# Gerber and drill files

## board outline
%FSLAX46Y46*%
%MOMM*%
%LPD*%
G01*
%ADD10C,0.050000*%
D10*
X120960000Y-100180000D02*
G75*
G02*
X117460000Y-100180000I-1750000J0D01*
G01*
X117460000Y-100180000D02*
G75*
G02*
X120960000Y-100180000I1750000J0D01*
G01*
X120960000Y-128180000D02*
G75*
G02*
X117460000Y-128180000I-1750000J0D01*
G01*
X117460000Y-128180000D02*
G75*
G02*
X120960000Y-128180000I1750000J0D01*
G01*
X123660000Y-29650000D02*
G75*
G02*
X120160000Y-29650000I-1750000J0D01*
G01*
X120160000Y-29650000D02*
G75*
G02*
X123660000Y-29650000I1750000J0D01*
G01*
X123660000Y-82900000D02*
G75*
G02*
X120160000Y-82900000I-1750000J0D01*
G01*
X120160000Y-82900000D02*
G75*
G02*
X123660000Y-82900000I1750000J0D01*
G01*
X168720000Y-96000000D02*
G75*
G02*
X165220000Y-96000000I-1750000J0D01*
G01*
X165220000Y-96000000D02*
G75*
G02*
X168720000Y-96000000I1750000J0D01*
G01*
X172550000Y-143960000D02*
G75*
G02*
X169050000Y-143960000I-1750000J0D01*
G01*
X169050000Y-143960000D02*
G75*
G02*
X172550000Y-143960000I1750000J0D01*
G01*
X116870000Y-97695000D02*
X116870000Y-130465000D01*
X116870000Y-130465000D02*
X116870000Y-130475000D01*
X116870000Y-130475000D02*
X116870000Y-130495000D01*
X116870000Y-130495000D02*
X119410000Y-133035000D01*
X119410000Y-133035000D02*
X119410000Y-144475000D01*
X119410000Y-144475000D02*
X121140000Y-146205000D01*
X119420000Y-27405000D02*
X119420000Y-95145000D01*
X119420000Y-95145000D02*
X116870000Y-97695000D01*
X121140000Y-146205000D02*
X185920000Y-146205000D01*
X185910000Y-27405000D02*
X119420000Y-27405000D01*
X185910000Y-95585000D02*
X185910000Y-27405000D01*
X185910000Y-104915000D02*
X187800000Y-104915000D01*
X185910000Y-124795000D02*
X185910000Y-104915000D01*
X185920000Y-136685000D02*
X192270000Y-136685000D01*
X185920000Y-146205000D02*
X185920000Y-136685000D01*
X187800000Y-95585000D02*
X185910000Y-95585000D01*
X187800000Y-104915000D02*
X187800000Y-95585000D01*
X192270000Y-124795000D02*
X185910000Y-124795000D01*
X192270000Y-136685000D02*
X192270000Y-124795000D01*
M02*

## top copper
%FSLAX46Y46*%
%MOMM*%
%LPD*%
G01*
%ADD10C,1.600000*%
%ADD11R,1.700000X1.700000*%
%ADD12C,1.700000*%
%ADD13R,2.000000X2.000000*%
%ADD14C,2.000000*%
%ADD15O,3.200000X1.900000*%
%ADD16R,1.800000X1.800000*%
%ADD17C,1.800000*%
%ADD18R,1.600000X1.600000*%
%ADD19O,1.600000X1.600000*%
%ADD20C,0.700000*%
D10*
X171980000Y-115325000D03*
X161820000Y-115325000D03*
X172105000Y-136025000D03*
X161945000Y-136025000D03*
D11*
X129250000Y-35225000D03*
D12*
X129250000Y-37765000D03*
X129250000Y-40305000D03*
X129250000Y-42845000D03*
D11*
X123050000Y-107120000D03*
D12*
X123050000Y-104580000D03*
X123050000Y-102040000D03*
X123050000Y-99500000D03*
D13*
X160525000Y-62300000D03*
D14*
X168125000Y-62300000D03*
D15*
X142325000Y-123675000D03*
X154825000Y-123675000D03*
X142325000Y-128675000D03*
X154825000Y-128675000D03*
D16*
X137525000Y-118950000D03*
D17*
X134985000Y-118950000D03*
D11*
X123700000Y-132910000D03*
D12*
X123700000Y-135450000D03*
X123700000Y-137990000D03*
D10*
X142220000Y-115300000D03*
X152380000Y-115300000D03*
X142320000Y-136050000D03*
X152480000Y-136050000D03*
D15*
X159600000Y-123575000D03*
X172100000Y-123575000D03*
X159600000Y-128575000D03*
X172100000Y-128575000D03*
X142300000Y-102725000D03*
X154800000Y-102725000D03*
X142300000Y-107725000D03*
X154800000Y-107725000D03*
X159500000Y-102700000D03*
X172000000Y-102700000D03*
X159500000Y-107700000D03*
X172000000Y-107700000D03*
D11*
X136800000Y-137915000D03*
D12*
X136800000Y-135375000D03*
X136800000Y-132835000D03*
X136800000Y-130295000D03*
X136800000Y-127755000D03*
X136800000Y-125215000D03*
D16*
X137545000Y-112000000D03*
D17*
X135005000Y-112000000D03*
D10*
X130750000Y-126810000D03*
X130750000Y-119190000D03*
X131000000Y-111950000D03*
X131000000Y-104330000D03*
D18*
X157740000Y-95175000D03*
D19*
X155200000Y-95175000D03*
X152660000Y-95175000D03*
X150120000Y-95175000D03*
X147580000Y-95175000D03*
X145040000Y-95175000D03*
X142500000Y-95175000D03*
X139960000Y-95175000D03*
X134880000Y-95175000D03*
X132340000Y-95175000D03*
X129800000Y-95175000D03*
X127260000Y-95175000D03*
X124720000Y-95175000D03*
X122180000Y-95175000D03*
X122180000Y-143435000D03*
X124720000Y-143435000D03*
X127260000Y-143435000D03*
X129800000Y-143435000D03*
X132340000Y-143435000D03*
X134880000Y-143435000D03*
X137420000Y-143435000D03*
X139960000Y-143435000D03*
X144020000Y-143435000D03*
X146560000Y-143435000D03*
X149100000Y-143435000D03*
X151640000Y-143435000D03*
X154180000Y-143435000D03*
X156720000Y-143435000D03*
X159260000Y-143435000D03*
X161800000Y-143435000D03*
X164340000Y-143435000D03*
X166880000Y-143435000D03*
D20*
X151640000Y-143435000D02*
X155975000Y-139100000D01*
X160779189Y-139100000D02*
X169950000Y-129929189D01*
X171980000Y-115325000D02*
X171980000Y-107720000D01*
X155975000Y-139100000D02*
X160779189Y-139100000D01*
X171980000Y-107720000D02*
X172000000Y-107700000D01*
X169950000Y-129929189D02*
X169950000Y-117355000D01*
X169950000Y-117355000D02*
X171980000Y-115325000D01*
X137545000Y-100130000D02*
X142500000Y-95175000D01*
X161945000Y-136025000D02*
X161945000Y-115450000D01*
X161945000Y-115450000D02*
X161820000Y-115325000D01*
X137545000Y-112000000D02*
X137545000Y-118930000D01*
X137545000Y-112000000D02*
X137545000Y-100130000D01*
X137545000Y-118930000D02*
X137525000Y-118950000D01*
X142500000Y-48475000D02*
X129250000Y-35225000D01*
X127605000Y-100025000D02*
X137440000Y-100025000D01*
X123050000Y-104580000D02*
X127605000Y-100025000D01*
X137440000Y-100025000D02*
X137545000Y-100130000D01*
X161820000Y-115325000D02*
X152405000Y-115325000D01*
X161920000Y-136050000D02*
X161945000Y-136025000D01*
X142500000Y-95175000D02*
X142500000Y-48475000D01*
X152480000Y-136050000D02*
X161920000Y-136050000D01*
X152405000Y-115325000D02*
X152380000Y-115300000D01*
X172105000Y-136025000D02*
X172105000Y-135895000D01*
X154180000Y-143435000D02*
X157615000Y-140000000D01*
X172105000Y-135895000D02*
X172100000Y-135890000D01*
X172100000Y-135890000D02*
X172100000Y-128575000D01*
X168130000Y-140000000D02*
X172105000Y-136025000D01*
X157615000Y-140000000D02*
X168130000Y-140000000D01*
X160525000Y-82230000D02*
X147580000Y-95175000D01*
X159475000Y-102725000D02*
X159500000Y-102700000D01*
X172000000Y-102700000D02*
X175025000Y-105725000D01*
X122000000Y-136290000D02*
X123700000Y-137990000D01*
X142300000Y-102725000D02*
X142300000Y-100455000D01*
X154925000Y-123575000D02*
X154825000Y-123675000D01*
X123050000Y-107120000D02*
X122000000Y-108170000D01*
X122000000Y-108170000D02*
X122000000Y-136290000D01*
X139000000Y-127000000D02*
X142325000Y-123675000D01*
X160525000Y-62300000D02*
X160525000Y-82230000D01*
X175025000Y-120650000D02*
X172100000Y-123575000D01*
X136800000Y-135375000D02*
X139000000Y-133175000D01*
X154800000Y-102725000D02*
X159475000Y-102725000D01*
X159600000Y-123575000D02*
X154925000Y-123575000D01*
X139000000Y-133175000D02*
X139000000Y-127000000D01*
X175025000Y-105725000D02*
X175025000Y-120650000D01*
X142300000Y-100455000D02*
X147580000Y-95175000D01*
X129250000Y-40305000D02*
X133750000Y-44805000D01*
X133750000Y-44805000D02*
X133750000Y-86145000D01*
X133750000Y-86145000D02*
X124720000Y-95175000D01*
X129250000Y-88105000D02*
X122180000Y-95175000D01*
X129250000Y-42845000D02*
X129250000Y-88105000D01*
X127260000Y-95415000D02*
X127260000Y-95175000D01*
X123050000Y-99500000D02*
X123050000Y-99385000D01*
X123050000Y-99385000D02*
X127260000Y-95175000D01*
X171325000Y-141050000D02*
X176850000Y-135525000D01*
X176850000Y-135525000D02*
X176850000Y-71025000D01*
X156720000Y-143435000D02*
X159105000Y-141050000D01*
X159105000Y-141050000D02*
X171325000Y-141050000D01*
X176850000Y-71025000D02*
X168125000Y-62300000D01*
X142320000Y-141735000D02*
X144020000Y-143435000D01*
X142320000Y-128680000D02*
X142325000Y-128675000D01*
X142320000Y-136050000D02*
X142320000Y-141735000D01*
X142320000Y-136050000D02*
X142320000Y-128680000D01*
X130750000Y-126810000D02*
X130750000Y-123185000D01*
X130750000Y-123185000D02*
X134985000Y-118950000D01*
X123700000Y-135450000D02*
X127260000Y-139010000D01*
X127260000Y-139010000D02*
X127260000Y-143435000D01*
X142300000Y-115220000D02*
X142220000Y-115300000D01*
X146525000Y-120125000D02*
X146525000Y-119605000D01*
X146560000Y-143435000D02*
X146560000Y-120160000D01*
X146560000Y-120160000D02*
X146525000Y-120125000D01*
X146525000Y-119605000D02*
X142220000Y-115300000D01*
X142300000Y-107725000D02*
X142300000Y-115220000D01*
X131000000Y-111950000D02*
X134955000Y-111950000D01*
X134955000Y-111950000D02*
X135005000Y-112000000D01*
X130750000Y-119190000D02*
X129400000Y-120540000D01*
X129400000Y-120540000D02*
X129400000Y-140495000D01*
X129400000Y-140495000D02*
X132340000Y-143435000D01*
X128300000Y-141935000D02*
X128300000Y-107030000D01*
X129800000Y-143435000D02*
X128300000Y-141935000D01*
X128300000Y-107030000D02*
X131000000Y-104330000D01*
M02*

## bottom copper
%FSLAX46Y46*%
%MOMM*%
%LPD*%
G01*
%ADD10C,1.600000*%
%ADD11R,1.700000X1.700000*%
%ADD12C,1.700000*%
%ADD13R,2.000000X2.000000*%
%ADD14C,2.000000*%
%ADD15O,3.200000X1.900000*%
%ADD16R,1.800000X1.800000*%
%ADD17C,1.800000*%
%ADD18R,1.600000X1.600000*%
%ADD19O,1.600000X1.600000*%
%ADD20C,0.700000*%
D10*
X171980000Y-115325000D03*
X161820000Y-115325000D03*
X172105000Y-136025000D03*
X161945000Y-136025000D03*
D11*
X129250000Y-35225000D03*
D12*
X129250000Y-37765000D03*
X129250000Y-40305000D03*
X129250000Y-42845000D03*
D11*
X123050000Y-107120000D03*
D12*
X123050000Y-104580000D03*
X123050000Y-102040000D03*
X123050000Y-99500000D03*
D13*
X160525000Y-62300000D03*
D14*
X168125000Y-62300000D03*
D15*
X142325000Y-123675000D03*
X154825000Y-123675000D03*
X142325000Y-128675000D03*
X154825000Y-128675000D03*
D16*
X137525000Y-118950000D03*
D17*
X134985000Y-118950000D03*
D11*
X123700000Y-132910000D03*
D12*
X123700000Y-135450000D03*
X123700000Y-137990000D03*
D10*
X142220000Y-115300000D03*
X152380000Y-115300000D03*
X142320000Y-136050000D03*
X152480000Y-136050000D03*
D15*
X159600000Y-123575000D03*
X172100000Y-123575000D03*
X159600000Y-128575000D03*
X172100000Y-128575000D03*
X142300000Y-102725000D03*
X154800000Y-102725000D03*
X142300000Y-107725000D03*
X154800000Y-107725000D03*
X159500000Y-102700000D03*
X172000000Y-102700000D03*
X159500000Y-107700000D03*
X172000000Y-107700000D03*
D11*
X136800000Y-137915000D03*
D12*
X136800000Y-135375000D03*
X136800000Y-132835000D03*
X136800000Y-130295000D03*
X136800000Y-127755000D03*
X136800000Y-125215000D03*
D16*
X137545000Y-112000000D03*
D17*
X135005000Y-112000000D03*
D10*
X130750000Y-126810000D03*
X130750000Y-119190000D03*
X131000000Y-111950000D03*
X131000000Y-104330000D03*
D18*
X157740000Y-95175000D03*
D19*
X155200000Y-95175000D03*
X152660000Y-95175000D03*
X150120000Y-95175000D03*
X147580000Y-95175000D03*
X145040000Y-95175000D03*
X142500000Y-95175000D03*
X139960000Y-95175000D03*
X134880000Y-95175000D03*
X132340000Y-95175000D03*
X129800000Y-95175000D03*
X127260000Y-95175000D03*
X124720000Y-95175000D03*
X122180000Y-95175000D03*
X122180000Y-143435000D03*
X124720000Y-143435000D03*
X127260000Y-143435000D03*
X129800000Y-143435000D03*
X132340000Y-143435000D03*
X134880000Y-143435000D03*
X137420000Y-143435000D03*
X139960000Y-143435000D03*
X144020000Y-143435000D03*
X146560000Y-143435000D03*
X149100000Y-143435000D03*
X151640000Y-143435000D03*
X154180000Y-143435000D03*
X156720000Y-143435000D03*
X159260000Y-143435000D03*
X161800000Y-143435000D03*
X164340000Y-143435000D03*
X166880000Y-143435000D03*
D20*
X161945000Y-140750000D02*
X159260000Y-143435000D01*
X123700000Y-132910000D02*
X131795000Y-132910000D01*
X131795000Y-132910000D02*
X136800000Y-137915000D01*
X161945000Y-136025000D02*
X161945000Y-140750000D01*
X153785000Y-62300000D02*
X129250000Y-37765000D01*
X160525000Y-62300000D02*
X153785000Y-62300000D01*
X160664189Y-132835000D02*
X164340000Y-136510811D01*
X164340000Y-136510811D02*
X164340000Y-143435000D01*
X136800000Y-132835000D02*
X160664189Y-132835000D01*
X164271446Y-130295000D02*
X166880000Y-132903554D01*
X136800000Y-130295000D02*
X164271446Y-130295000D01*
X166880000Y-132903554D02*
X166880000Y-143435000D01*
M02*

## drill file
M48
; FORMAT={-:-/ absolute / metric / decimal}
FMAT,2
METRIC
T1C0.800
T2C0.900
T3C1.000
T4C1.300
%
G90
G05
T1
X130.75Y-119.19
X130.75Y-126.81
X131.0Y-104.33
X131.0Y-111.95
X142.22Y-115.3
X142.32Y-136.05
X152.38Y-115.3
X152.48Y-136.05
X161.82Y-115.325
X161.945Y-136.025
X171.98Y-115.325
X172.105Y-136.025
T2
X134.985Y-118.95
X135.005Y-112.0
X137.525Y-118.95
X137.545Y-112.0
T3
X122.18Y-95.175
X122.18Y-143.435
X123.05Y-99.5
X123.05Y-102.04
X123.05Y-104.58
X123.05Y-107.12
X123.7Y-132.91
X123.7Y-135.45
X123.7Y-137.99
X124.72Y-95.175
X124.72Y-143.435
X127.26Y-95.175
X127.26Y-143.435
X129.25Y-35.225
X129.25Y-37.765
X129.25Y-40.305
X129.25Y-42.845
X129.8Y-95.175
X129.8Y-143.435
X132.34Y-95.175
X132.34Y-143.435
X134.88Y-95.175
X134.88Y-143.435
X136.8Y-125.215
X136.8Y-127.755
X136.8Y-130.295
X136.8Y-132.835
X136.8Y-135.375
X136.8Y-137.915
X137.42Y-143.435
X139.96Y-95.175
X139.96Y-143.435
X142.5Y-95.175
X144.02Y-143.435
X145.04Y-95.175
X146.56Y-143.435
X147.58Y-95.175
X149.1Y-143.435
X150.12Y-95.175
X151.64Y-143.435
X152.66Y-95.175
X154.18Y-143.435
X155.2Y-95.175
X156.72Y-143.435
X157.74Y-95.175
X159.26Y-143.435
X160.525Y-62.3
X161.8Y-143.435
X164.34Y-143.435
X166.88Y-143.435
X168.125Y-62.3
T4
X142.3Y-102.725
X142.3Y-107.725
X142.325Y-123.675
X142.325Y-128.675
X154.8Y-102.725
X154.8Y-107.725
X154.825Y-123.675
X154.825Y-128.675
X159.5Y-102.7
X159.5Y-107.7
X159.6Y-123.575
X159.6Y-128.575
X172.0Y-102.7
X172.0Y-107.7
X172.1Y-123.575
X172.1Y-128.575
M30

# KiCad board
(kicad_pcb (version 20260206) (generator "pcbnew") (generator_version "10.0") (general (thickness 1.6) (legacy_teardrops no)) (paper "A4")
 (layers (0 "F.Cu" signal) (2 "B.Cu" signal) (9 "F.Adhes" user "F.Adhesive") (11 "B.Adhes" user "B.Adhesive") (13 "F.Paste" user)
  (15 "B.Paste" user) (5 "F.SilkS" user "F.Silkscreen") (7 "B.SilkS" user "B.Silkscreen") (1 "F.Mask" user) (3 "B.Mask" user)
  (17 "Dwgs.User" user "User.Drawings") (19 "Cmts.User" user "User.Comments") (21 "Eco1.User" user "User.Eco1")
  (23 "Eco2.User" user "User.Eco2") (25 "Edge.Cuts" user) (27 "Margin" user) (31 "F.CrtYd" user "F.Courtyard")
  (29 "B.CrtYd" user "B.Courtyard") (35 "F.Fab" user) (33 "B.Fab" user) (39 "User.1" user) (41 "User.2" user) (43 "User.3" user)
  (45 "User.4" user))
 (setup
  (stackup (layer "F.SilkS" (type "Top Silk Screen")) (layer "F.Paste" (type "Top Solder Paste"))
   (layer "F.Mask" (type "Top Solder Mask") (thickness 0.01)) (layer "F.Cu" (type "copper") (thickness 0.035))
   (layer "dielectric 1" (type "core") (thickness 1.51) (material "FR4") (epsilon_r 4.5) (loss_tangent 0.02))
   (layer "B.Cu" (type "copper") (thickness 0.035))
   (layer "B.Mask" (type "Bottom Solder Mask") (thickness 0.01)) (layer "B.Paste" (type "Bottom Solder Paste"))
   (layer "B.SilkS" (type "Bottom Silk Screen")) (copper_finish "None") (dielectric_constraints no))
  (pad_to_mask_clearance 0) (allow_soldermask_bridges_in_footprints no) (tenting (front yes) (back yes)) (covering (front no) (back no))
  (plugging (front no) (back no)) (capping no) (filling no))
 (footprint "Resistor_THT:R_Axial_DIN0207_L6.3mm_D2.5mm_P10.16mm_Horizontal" (layer "F.Cu") (at 171.98 115.325 180)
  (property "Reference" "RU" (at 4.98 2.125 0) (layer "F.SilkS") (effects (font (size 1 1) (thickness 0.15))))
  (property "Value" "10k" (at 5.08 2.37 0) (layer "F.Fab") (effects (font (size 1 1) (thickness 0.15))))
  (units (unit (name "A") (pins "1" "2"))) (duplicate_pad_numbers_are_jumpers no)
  (pad "1" thru_hole circle (at 0 0 180) (size 1.6 1.6) (drill 0.8) (layers "*.Cu" "*.Mask") (remove_unused_layers no) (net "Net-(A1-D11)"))
  (pad "2" thru_hole circle (at 10.16 0 180) (size 1.6 1.6) (drill 0.8) (layers "*.Cu" "*.Mask") (remove_unused_layers no) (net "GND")))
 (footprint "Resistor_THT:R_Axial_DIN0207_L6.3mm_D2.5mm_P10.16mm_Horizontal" (layer "F.Cu") (at 172.105 136.025 180)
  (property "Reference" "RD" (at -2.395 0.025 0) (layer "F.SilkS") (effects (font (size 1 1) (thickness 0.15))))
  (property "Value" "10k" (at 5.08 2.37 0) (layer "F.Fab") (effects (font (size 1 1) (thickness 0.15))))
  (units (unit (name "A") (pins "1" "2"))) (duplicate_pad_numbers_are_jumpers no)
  (pad "1" thru_hole circle (at 0 0 180) (size 1.6 1.6) (drill 0.8) (layers "*.Cu" "*.Mask") (remove_unused_layers no) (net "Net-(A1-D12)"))
  (pad "2" thru_hole circle (at 10.16 0 180) (size 1.6 1.6) (drill 0.8) (layers "*.Cu" "*.Mask") (remove_unused_layers no) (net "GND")))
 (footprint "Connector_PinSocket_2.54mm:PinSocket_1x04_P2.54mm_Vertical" (layer "F.Cu") (at 129.25 35.225)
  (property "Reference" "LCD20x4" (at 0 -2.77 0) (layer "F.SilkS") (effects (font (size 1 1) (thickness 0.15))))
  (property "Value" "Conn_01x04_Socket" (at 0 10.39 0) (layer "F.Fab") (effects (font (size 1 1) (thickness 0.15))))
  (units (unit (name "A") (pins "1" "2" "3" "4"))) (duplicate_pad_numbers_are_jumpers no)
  (pad "1" thru_hole rect (at 0 0) (size 1.7 1.7) (drill 1) (layers "*.Cu" "*.Mask") (remove_unused_layers no) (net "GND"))
  (pad "2" thru_hole circle (at 0 2.54) (size 1.7 1.7) (drill 1) (layers "*.Cu" "*.Mask") (remove_unused_layers no) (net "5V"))
  (pad "3" thru_hole circle (at 0 5.08) (size 1.7 1.7) (drill 1) (layers "*.Cu" "*.Mask") (remove_unused_layers no)
   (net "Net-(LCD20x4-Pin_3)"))
  (pad "4" thru_hole circle (at 0 7.62) (size 1.7 1.7) (drill 1) (layers "*.Cu" "*.Mask") (remove_unused_layers no)
   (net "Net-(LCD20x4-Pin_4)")))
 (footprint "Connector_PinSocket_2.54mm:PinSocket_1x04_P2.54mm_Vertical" (layer "F.Cu") (at 123.05 107.12 180)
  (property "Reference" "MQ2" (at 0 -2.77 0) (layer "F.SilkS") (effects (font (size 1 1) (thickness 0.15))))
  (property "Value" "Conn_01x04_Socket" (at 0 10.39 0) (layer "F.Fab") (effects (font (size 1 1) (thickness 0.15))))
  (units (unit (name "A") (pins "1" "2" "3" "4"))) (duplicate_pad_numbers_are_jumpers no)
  (pad "1" thru_hole rect (at 0 0 180) (size 1.7 1.7) (drill 1) (layers "*.Cu" "*.Mask") (remove_unused_layers no) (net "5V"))
  (pad "2" thru_hole circle (at 0 2.54 180) (size 1.7 1.7) (drill 1) (layers "*.Cu" "*.Mask") (remove_unused_layers no) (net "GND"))
  (pad "3" thru_hole circle (at 0 5.08 180) (size 1.7 1.7) (drill 1) (layers "*.Cu" "*.Mask") (remove_unused_layers no)
   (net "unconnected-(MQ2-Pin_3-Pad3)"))
  (pad "4" thru_hole circle (at 0 7.62 180) (size 1.7 1.7) (drill 1) (layers "*.Cu" "*.Mask") (remove_unused_layers no) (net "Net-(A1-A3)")))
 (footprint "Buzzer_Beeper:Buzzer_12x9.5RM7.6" (layer "F.Cu") (at 160.525 62.3)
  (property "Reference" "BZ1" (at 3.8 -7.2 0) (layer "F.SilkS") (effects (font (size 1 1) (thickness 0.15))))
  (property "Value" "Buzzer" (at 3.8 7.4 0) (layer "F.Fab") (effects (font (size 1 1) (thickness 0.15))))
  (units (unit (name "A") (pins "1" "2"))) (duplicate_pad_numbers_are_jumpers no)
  (pad "1" thru_hole rect (at 0 0) (size 2 2) (drill 1) (layers "*.Cu" "*.Mask") (remove_unused_layers no) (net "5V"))
  (pad "2" thru_hole circle (at 7.6 0) (size 2 2) (drill 1) (layers "*.Cu" "*.Mask") (remove_unused_layers no) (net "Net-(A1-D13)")))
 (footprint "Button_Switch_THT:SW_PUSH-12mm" (layer "F.Cu") (at 142.325 123.675)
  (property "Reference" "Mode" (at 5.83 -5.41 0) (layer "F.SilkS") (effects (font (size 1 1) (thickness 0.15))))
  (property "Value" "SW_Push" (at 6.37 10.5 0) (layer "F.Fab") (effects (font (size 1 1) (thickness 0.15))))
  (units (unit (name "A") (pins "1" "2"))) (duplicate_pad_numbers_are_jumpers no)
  (pad "1" thru_hole oval (at 0 0) (size 3.2 1.9) (drill 1.3) (layers "*.Cu" "*.Mask") (remove_unused_layers no) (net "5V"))
  (pad "1" thru_hole oval (at 12.5 0) (size 3.2 1.9) (drill 1.3) (layers "*.Cu" "*.Mask") (remove_unused_layers no) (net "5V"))
  (pad "2" thru_hole oval (at 0 5) (size 3.2 1.9) (drill 1.3) (layers "*.Cu" "*.Mask") (remove_unused_layers no) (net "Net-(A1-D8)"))
  (pad "2" thru_hole oval (at 12.5 5) (size 3.2 1.9) (drill 1.3) (layers "*.Cu" "*.Mask") (remove_unused_layers no) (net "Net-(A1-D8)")))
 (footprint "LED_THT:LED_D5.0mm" (layer "F.Cu") (at 137.525 118.95 180)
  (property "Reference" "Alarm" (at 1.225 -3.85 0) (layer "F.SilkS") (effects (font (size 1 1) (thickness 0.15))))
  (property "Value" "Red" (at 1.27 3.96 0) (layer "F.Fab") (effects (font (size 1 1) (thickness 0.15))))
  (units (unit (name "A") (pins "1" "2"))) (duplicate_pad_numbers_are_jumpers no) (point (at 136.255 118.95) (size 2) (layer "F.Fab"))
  (pad "1" thru_hole rect (at 0 0 180) (size 1.8 1.8) (drill 0.9) (layers "*.Cu" "*.Mask") (remove_unused_layers no) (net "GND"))
  (pad "2" thru_hole circle (at 2.54 0 180) (size 1.8 1.8) (drill 0.9) (layers "*.Cu" "*.Mask") (remove_unused_layers no)
   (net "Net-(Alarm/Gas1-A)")))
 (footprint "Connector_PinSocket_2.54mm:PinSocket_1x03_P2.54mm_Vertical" (layer "F.Cu") (at 123.7 132.91)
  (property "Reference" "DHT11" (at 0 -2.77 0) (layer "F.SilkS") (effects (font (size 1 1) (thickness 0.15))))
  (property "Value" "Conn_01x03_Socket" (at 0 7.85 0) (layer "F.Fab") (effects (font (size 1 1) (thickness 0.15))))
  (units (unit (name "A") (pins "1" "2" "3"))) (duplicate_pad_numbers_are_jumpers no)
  (pad "1" thru_hole rect (at 0 0) (size 1.7 1.7) (drill 1) (layers "*.Cu" "*.Mask") (remove_unused_layers no) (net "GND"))
  (pad "2" thru_hole circle (at 0 2.54) (size 1.7 1.7) (drill 1) (layers "*.Cu" "*.Mask") (remove_unused_layers no) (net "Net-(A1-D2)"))
  (pad "3" thru_hole circle (at 0 5.08) (size 1.7 1.7) (drill 1) (layers "*.Cu" "*.Mask") (remove_unused_layers no) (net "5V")))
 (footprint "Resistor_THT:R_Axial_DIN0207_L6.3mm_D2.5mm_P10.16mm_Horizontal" (layer "F.Cu") (at 142.22 115.3)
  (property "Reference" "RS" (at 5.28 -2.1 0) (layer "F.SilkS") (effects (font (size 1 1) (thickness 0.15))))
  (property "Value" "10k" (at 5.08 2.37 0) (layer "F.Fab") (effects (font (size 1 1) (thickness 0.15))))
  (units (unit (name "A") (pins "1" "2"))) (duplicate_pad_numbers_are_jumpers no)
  (pad "1" thru_hole circle (at 0 0) (size 1.6 1.6) (drill 0.8) (layers "*.Cu" "*.Mask") (remove_unused_layers no) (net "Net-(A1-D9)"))
  (pad "2" thru_hole circle (at 10.16 0) (size 1.6 1.6) (drill 0.8) (layers "*.Cu" "*.Mask") (remove_unused_layers no) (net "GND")))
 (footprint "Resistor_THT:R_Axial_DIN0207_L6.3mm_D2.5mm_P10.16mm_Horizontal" (layer "F.Cu") (at 142.32 136.05)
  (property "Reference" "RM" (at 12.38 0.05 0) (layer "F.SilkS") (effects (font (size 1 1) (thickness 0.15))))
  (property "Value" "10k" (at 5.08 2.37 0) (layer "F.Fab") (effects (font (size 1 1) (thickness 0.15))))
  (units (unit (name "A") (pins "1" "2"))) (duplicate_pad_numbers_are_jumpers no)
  (pad "1" thru_hole circle (at 0 0) (size 1.6 1.6) (drill 0.8) (layers "*.Cu" "*.Mask") (remove_unused_layers no) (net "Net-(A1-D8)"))
  (pad "2" thru_hole circle (at 10.16 0) (size 1.6 1.6) (drill 0.8) (layers "*.Cu" "*.Mask") (remove_unused_layers no) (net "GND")))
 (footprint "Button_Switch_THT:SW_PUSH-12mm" (layer "F.Cu") (at 159.6 123.575)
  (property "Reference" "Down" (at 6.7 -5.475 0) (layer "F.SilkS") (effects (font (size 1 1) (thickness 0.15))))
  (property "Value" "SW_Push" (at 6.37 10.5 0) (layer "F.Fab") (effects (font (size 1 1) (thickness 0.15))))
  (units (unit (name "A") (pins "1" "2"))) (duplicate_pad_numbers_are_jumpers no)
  (pad "1" thru_hole oval (at 0 0) (size 3.2 1.9) (drill 1.3) (layers "*.Cu" "*.Mask") (remove_unused_layers no) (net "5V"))
  (pad "1" thru_hole oval (at 12.5 0) (size 3.2 1.9) (drill 1.3) (layers "*.Cu" "*.Mask") (remove_unused_layers no) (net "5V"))
  (pad "2" thru_hole oval (at 0 5) (size 3.2 1.9) (drill 1.3) (layers "*.Cu" "*.Mask") (remove_unused_layers no) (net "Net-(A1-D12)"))
  (pad "2" thru_hole oval (at 12.5 5) (size 3.2 1.9) (drill 1.3) (layers "*.Cu" "*.Mask") (remove_unused_layers no) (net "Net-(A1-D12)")))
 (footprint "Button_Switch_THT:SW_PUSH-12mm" (layer "F.Cu") (at 142.3 102.725)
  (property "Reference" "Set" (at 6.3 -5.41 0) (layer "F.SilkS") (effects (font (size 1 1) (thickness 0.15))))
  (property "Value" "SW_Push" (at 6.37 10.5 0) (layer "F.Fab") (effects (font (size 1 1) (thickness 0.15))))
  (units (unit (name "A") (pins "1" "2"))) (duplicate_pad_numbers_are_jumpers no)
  (pad "1" thru_hole oval (at 0 0) (size 3.2 1.9) (drill 1.3) (layers "*.Cu" "*.Mask") (remove_unused_layers no) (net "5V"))
  (pad "1" thru_hole oval (at 12.5 0) (size 3.2 1.9) (drill 1.3) (layers "*.Cu" "*.Mask") (remove_unused_layers no) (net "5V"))
  (pad "2" thru_hole oval (at 0 5) (size 3.2 1.9) (drill 1.3) (layers "*.Cu" "*.Mask") (remove_unused_layers no) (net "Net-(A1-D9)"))
  (pad "2" thru_hole oval (at 12.5 5) (size 3.2 1.9) (drill 1.3) (layers "*.Cu" "*.Mask") (remove_unused_layers no) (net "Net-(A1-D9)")))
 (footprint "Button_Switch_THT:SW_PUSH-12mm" (layer "F.Cu") (at 159.5 102.7)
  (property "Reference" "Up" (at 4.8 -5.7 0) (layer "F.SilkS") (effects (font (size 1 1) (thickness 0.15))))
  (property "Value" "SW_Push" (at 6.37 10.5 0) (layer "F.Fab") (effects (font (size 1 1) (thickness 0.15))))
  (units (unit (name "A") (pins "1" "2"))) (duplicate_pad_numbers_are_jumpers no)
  (pad "1" thru_hole oval (at 0 0) (size 3.2 1.9) (drill 1.3) (layers "*.Cu" "*.Mask") (remove_unused_layers no) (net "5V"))
  (pad "1" thru_hole oval (at 12.5 0) (size 3.2 1.9) (drill 1.3) (layers "*.Cu" "*.Mask") (remove_unused_layers no) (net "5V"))
  (pad "2" thru_hole oval (at 0 5) (size 3.2 1.9) (drill 1.3) (layers "*.Cu" "*.Mask") (remove_unused_layers no) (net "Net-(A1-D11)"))
  (pad "2" thru_hole oval (at 12.5 5) (size 3.2 1.9) (drill 1.3) (layers "*.Cu" "*.Mask") (remove_unused_layers no) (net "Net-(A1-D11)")))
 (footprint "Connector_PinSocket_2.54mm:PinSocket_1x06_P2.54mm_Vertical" (layer "F.Cu") (at 136.8 137.915 180)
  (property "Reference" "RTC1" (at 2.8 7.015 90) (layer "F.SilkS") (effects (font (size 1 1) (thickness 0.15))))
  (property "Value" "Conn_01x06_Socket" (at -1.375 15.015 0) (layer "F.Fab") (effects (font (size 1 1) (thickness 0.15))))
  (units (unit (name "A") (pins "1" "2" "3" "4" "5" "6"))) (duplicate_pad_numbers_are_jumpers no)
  (pad "1" thru_hole rect (at 0 0 180) (size 1.7 1.7) (drill 1) (layers "*.Cu" "*.Mask") (remove_unused_layers no) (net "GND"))
  (pad "2" thru_hole circle (at 0 2.54 180) (size 1.7 1.7) (drill 1) (layers "*.Cu" "*.Mask") (remove_unused_layers no) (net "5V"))
  (pad "3" thru_hole circle (at 0 5.08 180) (size 1.7 1.7) (drill 1) (layers "*.Cu" "*.Mask") (remove_unused_layers no)
   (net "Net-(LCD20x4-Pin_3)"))
  (pad "4" thru_hole circle (at 0 7.62 180) (size 1.7 1.7) (drill 1) (layers "*.Cu" "*.Mask") (remove_unused_layers no)
   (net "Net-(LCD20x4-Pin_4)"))
  (pad "5" thru_hole circle (at 0 10.16 180) (size 1.7 1.7) (drill 1) (layers "*.Cu" "*.Mask") (remove_unused_layers no)
   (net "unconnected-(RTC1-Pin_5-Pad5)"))
  (pad "6" thru_hole circle (at 0 12.7 180) (size 1.7 1.7) (drill 1) (layers "*.Cu" "*.Mask") (remove_unused_layers no)
   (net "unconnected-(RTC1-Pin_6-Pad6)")))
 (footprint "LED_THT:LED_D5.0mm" (layer "F.Cu") (at 137.545 112 180)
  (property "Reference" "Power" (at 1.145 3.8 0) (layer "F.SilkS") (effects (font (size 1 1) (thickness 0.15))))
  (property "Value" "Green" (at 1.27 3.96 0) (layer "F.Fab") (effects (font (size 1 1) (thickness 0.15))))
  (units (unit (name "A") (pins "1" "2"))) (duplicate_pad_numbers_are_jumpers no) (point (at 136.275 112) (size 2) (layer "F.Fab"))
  (pad "1" thru_hole rect (at 0 0 180) (size 1.8 1.8) (drill 0.9) (layers "*.Cu" "*.Mask") (remove_unused_layers no) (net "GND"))
  (pad "2" thru_hole circle (at 2.54 0 180) (size 1.8 1.8) (drill 0.9) (layers "*.Cu" "*.Mask") (remove_unused_layers no)
   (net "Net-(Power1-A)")))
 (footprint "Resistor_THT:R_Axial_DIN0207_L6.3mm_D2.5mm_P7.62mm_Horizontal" (layer "F.Cu") (at 130.75 126.81 90)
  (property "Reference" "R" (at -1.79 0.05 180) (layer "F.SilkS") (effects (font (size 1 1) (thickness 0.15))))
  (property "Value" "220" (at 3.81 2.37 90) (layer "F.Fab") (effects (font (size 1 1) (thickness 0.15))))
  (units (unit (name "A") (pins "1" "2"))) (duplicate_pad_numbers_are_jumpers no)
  (pad "1" thru_hole circle (at 0 0 90) (size 1.6 1.6) (drill 0.8) (layers "*.Cu" "*.Mask") (remove_unused_layers no)
   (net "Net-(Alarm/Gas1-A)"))
  (pad "2" thru_hole circle (at 7.62 0 90) (size 1.6 1.6) (drill 0.8) (layers "*.Cu" "*.Mask") (remove_unused_layers no) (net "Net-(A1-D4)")))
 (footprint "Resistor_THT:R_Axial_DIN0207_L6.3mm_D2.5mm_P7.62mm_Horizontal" (layer "F.Cu") (at 131 111.95 90)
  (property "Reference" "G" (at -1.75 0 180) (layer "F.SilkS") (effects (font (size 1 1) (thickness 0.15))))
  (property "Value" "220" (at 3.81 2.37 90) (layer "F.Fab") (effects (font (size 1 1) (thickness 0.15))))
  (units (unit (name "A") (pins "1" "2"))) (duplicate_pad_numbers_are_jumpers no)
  (pad "1" thru_hole circle (at 0 0 90) (size 1.6 1.6) (drill 0.8) (layers "*.Cu" "*.Mask") (remove_unused_layers no) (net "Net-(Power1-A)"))
  (pad "2" thru_hole circle (at 7.62 0 90) (size 1.6 1.6) (drill 0.8) (layers "*.Cu" "*.Mask") (remove_unused_layers no) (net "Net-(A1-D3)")))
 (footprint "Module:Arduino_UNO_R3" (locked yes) (layer "B.Cu") (at 157.74 95.175 180)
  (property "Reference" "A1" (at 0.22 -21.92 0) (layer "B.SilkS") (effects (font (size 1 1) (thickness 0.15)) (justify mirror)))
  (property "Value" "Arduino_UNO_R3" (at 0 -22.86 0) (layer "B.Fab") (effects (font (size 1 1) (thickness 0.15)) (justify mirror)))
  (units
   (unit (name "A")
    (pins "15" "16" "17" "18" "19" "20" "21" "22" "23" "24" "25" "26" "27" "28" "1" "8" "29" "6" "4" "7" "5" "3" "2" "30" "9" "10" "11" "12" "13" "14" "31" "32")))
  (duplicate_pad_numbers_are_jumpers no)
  (fp_line (start 40.87 -2.52) (end 40.87 -35.29) (stroke (width 0.05) (type default)) (layer "Edge.Cuts"))
  (fp_line (start 40.87 -35.29) (end 40.87 -35.3) (stroke (width 0.05) (type default)) (layer "Edge.Cuts"))
  (fp_line (start 40.87 -35.3) (end 40.87 -35.32) (stroke (width 0.05) (type default)) (layer "Edge.Cuts"))
  (fp_line (start 40.87 -35.32) (end 38.33 -37.86) (stroke (width 0.05) (type default)) (layer "Edge.Cuts"))
  (fp_line (start 38.33 -37.86) (end 38.33 -49.3) (stroke (width 0.05) (type default)) (layer "Edge.Cuts"))
  (fp_line (start 38.33 -49.3) (end 36.6 -51.03) (stroke (width 0.05) (type default)) (layer "Edge.Cuts"))
  (fp_line (start 38.32 67.77) (end 38.32 0.03) (stroke (width 0.05) (type default)) (layer "Edge.Cuts"))
  (fp_line (start 38.32 0.03) (end 40.87 -2.52) (stroke (width 0.05) (type default)) (layer "Edge.Cuts"))
  (fp_line (start 36.6 -51.03) (end -28.18 -51.03) (stroke (width 0.05) (type default)) (layer "Edge.Cuts"))
  (fp_line (start -28.17 67.77) (end 38.32 67.77) (stroke (width 0.05) (type default)) (layer "Edge.Cuts"))
  (fp_line (start -28.17 -0.41) (end -28.17 67.77) (stroke (width 0.05) (type default)) (layer "Edge.Cuts"))
  (fp_line (start -28.17 -9.74) (end -30.06 -9.74) (stroke (width 0.05) (type default)) (layer "Edge.Cuts"))
  (fp_line (start -28.17 -29.62) (end -28.17 -9.74) (stroke (width 0.05) (type default)) (layer "Edge.Cuts"))
  (fp_line (start -28.18 -41.51) (end -34.53 -41.51) (stroke (width 0.05) (type default)) (layer "Edge.Cuts"))
  (fp_line (start -28.18 -51.03) (end -28.18 -41.51) (stroke (width 0.05) (type default)) (layer "Edge.Cuts"))
  (fp_line (start -30.06 -0.41) (end -28.17 -0.41) (stroke (width 0.05) (type default)) (layer "Edge.Cuts"))
  (fp_line (start -30.06 -9.74) (end -30.06 -0.41) (stroke (width 0.05) (type default)) (layer "Edge.Cuts"))
  (fp_line (start -34.53 -29.62) (end -28.17 -29.62) (stroke (width 0.05) (type default)) (layer "Edge.Cuts"))
  (fp_line (start -34.53 -41.51) (end -34.53 -29.62) (stroke (width 0.05) (type default)) (layer "Edge.Cuts"))
  (pad "1" thru_hole rect (at 0 0 90) (size 1.6 1.6) (drill 1) (layers "*.Cu" "*.Mask") (remove_unused_layers no)
   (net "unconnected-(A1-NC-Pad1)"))
  (pad "2" thru_hole oval (at 2.54 0 90) (size 1.6 1.6) (drill 1) (layers "*.Cu" "*.Mask") (remove_unused_layers no)
   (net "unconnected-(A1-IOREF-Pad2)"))
  (pad "3" thru_hole oval (at 5.08 0 90) (size 1.6 1.6) (drill 1) (layers "*.Cu" "*.Mask") (remove_unused_layers no)
   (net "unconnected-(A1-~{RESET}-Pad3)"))
  (pad "4" thru_hole oval (at 7.62 0 90) (size 1.6 1.6) (drill 1) (layers "*.Cu" "*.Mask") (remove_unused_layers no)
   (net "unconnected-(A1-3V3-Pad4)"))
  (pad "5" thru_hole oval (at 10.16 0 90) (size 1.6 1.6) (drill 1) (layers "*.Cu" "*.Mask") (remove_unused_layers no) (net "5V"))
  (pad "6" thru_hole oval (at 12.7 0 90) (size 1.6 1.6) (drill 1) (layers "*.Cu" "*.Mask") (remove_unused_layers no) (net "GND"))
  (pad "7" thru_hole oval (at 15.24 0 90) (size 1.6 1.6) (drill 1) (layers "*.Cu" "*.Mask") (remove_unused_layers no) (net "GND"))
  (pad "8" thru_hole oval (at 17.78 0 90) (size 1.6 1.6) (drill 1) (layers "*.Cu" "*.Mask") (remove_unused_layers no)
   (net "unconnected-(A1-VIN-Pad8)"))
  (pad "9" thru_hole oval (at 22.86 0 90) (size 1.6 1.6) (drill 1) (layers "*.Cu" "*.Mask") (remove_unused_layers no)
   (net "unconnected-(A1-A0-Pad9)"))
  (pad "10" thru_hole oval (at 25.4 0 90) (size 1.6 1.6) (drill 1) (layers "*.Cu" "*.Mask") (remove_unused_layers no)
   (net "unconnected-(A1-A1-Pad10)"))
  (pad "11" thru_hole oval (at 27.94 0 90) (size 1.6 1.6) (drill 1) (layers "*.Cu" "*.Mask") (remove_unused_layers no)
   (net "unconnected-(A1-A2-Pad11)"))
  (pad "12" thru_hole oval (at 30.48 0 90) (size 1.6 1.6) (drill 1) (layers "*.Cu" "*.Mask") (remove_unused_layers no) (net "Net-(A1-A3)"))
  (pad "13" thru_hole oval (at 33.02 0 90) (size 1.6 1.6) (drill 1) (layers "*.Cu" "*.Mask") (remove_unused_layers no)
   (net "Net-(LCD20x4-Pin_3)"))
  (pad "14" thru_hole oval (at 35.56 0 90) (size 1.6 1.6) (drill 1) (layers "*.Cu" "*.Mask") (remove_unused_layers no)
   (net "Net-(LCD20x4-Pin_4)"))
  (pad "15" thru_hole oval (at 35.56 -48.26 90) (size 1.6 1.6) (drill 1) (layers "*.Cu" "*.Mask") (remove_unused_layers no)
   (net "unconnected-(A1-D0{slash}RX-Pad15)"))
  (pad "16" thru_hole oval (at 33.02 -48.26 90) (size 1.6 1.6) (drill 1) (layers "*.Cu" "*.Mask") (remove_unused_layers no)
   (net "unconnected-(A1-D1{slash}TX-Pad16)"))
  (pad "17" thru_hole oval (at 30.48 -48.26 90) (size 1.6 1.6) (drill 1) (layers "*.Cu" "*.Mask") (remove_unused_layers no)
   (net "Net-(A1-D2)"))
  (pad "18" thru_hole oval (at 27.94 -48.26 90) (size 1.6 1.6) (drill 1) (layers "*.Cu" "*.Mask") (remove_unused_layers no)
   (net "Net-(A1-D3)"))
  (pad "19" thru_hole oval (at 25.4 -48.26 90) (size 1.6 1.6) (drill 1) (layers "*.Cu" "*.Mask") (remove_unused_layers no)
   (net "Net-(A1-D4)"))
  (pad "20" thru_hole oval (at 22.86 -48.26 90) (size 1.6 1.6) (drill 1) (layers "*.Cu" "*.Mask") (remove_unused_layers no)
   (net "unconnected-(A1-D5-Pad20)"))
  (pad "21" thru_hole oval (at 20.32 -48.26 90) (size 1.6 1.6) (drill 1) (layers "*.Cu" "*.Mask") (remove_unused_layers no)
   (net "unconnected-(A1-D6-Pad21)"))
  (pad "22" thru_hole oval (at 17.78 -48.26 90) (size 1.6 1.6) (drill 1) (layers "*.Cu" "*.Mask") (remove_unused_layers no)
   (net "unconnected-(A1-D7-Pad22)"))
  (pad "23" thru_hole oval (at 13.72 -48.26 90) (size 1.6 1.6) (drill 1) (layers "*.Cu" "*.Mask") (remove_unused_layers no)
   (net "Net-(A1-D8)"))
  (pad "24" thru_hole oval (at 11.18 -48.26 90) (size 1.6 1.6) (drill 1) (layers "*.Cu" "*.Mask") (remove_unused_layers no)
   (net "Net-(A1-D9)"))
  (pad "25" thru_hole oval (at 8.64 -48.26 90) (size 1.6 1.6) (drill 1) (layers "*.Cu" "*.Mask") (remove_unused_layers no)
   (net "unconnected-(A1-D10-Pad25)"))
  (pad "26" thru_hole oval (at 6.1 -48.26 90) (size 1.6 1.6) (drill 1) (layers "*.Cu" "*.Mask") (remove_unused_layers no)
   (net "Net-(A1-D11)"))
  (pad "27" thru_hole oval (at 3.56 -48.26 90) (size 1.6 1.6) (drill 1) (layers "*.Cu" "*.Mask") (remove_unused_layers no)
   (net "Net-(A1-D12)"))
  (pad "28" thru_hole oval (at 1.02 -48.26 90) (size 1.6 1.6) (drill 1) (layers "*.Cu" "*.Mask") (remove_unused_layers no)
   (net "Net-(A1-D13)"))
  (pad "29" thru_hole oval (at -1.52 -48.26 90) (size 1.6 1.6) (drill 1) (layers "*.Cu" "*.Mask") (remove_unused_layers no) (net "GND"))
  (pad "30" thru_hole oval (at -4.06 -48.26 90) (size 1.6 1.6) (drill 1) (layers "*.Cu" "*.Mask") (remove_unused_layers no)
   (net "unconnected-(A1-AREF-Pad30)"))
  (pad "31" thru_hole oval (at -6.6 -48.26 90) (size 1.6 1.6) (drill 1) (layers "*.Cu" "*.Mask") (remove_unused_layers no)
   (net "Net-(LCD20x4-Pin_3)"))
  (pad "32" thru_hole oval (at -9.14 -48.26 90) (size 1.6 1.6) (drill 1) (layers "*.Cu" "*.Mask") (remove_unused_layers no)
   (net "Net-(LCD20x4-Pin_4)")))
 (gr_circle (center 119.21 100.18) (end 120.96 100.18) (stroke (width 0.05) (type default)) (fill no) (layer "Edge.Cuts"))
 (gr_circle (center 119.21 128.18) (end 120.96 128.18) (stroke (width 0.05) (type default)) (fill no) (layer "Edge.Cuts"))
 (gr_circle (center 121.91 29.65) (end 123.66 29.65) (stroke (width 0.05) (type default)) (fill no) (layer "Edge.Cuts"))
 (gr_circle (center 121.91 82.9) (end 123.66 82.9) (stroke (width 0.05) (type default)) (fill no) (layer "Edge.Cuts"))
 (gr_circle (center 166.97 96) (end 168.72 96) (stroke (width 0.05) (type default)) (fill no) (layer "Edge.Cuts"))
 (gr_circle (center 170.8 143.96) (end 172.55 143.96) (stroke (width 0.05) (type default)) (fill no) (layer "Edge.Cuts"))
 (segment (start 151.64 143.435) (end 155.975 139.1) (width 0.7) (layer "F.Cu") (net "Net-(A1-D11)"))
 (segment (start 160.779189 139.1) (end 169.95 129.929189) (width 0.7) (layer "F.Cu") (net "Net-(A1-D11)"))
 (segment (start 171.98 115.325) (end 171.98 107.72) (width 0.7) (layer "F.Cu") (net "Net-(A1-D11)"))
 (segment (start 155.975 139.1) (end 160.779189 139.1) (width 0.7) (layer "F.Cu") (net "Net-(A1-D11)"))
 (segment (start 171.98 107.72) (end 172 107.7) (width 0.7) (layer "F.Cu") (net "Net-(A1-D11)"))
 (segment (start 169.95 129.929189) (end 169.95 117.355) (width 0.7) (layer "F.Cu") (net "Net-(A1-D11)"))
 (segment (start 169.95 117.355) (end 171.98 115.325) (width 0.7) (layer "F.Cu") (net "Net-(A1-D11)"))
 (segment (start 137.545 100.13) (end 142.5 95.175) (width 0.7) (layer "F.Cu") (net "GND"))
 (segment (start 161.945 136.025) (end 161.945 115.45) (width 0.7) (layer "F.Cu") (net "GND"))
 (segment (start 161.945 115.45) (end 161.82 115.325) (width 0.7) (layer "F.Cu") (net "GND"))
 (segment (start 137.545 112) (end 137.545 118.93) (width 0.7) (layer "F.Cu") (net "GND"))
 (segment (start 137.545 112) (end 137.545 100.13) (width 0.7) (layer "F.Cu") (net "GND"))
 (segment (start 137.545 118.93) (end 137.525 118.95) (width 0.7) (layer "F.Cu") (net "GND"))
 (segment (start 142.5 48.475) (end 129.25 35.225) (width 0.7) (layer "F.Cu") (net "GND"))
 (segment (start 127.605 100.025) (end 137.44 100.025) (width 0.7) (layer "F.Cu") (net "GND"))
 (segment (start 123.05 104.58) (end 127.605 100.025) (width 0.7) (layer "F.Cu") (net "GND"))
 (segment (start 137.44 100.025) (end 137.545 100.13) (width 0.7) (layer "F.Cu") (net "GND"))
 (segment (start 161.82 115.325) (end 152.405 115.325) (width 0.7) (layer "F.Cu") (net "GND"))
 (segment (start 161.92 136.05) (end 161.945 136.025) (width 0.7) (layer "F.Cu") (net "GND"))
 (segment (start 142.5 95.175) (end 142.5 48.475) (width 0.7) (layer "F.Cu") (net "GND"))
 (segment (start 152.48 136.05) (end 161.92 136.05) (width 0.7) (layer "F.Cu") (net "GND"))
 (segment (start 152.405 115.325) (end 152.38 115.3) (width 0.7) (layer "F.Cu") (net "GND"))
 (segment (start 161.945 140.75) (end 159.26 143.435) (width 0.7) (layer "B.Cu") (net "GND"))
 (segment (start 123.7 132.91) (end 131.795 132.91) (width 0.7) (layer "B.Cu") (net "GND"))
 (segment (start 131.795 132.91) (end 136.8 137.915) (width 0.7) (layer "B.Cu") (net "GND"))
 (segment (start 161.945 136.025) (end 161.945 140.75) (width 0.7) (layer "B.Cu") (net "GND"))
 (segment (start 172.105 136.025) (end 172.105 135.895) (width 0.7) (layer "F.Cu") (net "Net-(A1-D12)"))
 (segment (start 154.18 143.435) (end 157.615 140) (width 0.7) (layer "F.Cu") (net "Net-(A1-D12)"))
 (segment (start 172.105 135.895) (end 172.1 135.89) (width 0.7) (layer "F.Cu") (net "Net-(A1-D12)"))
 (segment (start 172.1 135.89) (end 172.1 128.575) (width 0.7) (layer "F.Cu") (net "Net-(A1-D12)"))
 (segment (start 168.13 140) (end 172.105 136.025) (width 0.7) (layer "F.Cu") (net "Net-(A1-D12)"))
 (segment (start 157.615 140) (end 168.13 140) (width 0.7) (layer "F.Cu") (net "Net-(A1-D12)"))
 (segment (start 160.525 82.23) (end 147.58 95.175) (width 0.7) (layer "F.Cu") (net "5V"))
 (segment (start 159.475 102.725) (end 159.5 102.7) (width 0.7) (layer "F.Cu") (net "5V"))
 (segment (start 172 102.7) (end 175.025 105.725) (width 0.7) (layer "F.Cu") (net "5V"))
 (segment (start 122 136.29) (end 123.7 137.99) (width 0.7) (layer "F.Cu") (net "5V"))
 (segment (start 142.3 102.725) (end 142.3 100.455) (width 0.7) (layer "F.Cu") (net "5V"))
 (segment (start 154.925 123.575) (end 154.825 123.675) (width 0.7) (layer "F.Cu") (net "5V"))
 (segment (start 123.05 107.12) (end 122 108.17) (width 0.7) (layer "F.Cu") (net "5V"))
 (segment (start 122 108.17) (end 122 136.29) (width 0.7) (layer "F.Cu") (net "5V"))
 (segment (start 139 127) (end 142.325 123.675) (width 0.7) (layer "F.Cu") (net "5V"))
 (segment (start 160.525 62.3) (end 160.525 82.23) (width 0.7) (layer "F.Cu") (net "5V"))
 (segment (start 175.025 120.65) (end 172.1 123.575) (width 0.7) (layer "F.Cu") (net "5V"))
 (segment (start 136.8 135.375) (end 139 133.175) (width 0.7) (layer "F.Cu") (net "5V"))
 (segment (start 154.8 102.725) (end 159.475 102.725) (width 0.7) (layer "F.Cu") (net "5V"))
 (segment (start 159.6 123.575) (end 154.925 123.575) (width 0.7) (layer "F.Cu") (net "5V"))
 (segment (start 139 133.175) (end 139 127) (width 0.7) (layer "F.Cu") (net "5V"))
 (segment (start 175.025 105.725) (end 175.025 120.65) (width 0.7) (layer "F.Cu") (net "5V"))
 (segment (start 142.3 100.455) (end 147.58 95.175) (width 0.7) (layer "F.Cu") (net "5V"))
 (segment (start 153.785 62.3) (end 129.25 37.765) (width 0.7) (layer "B.Cu") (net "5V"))
 (segment (start 160.525 62.3) (end 153.785 62.3) (width 0.7) (layer "B.Cu") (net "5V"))
 (segment (start 129.25 40.305) (end 133.75 44.805) (width 0.7) (layer "F.Cu") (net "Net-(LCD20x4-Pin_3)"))
 (segment (start 133.75 44.805) (end 133.75 86.145) (width 0.7) (layer "F.Cu") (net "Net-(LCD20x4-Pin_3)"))
 (segment (start 133.75 86.145) (end 124.72 95.175) (width 0.7) (layer "F.Cu") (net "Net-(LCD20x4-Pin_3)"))
 (segment (start 160.664189 132.835) (end 164.34 136.510811) (width 0.7) (layer "B.Cu") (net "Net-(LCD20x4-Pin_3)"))
 (segment (start 164.34 136.510811) (end 164.34 143.435) (width 0.7) (layer "B.Cu") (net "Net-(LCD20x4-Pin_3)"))
 (segment (start 136.8 132.835) (end 160.664189 132.835) (width 0.7) (layer "B.Cu") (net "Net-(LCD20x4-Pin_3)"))
 (segment (start 129.25 88.105) (end 122.18 95.175) (width 0.7) (layer "F.Cu") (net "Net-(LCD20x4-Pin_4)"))
 (segment (start 129.25 42.845) (end 129.25 88.105) (width 0.7) (layer "F.Cu") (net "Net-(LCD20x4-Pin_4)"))
 (segment (start 164.271446 130.295) (end 166.88 132.903554) (width 0.7) (layer "B.Cu") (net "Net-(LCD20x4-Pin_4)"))
 (segment (start 136.8 130.295) (end 164.271446 130.295) (width 0.7) (layer "B.Cu") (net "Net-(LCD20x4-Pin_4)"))
 (segment (start 166.88 132.903554) (end 166.88 143.435) (width 0.7) (layer "B.Cu") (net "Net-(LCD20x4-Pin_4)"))
 (segment (start 127.26 95.415) (end 127.26 95.175) (width 0.7) (layer "F.Cu") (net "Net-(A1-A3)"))
 (segment (start 123.05 99.5) (end 123.05 99.385) (width 0.7) (layer "F.Cu") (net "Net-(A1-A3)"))
 (segment (start 123.05 99.385) (end 127.26 95.175) (width 0.7) (layer "F.Cu") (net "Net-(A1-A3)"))
 (segment (start 171.325 141.05) (end 176.85 135.525) (width 0.7) (layer "F.Cu") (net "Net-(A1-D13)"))
 (segment (start 176.85 135.525) (end 176.85 71.025) (width 0.7) (layer "F.Cu") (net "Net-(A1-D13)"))
 (segment (start 156.72 143.435) (end 159.105 141.05) (width 0.7) (layer "F.Cu") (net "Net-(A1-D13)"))
 (segment (start 159.105 141.05) (end 171.325 141.05) (width 0.7) (layer "F.Cu") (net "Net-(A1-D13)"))
 (segment (start 176.85 71.025) (end 168.125 62.3) (width 0.7) (layer "F.Cu") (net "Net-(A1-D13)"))
 (segment (start 142.32 141.735) (end 144.02 143.435) (width 0.7) (layer "F.Cu") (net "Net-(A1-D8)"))
 (segment (start 142.32 128.68) (end 142.325 128.675) (width 0.7) (layer "F.Cu") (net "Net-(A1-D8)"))
 (segment (start 142.32 136.05) (end 142.32 141.735) (width 0.7) (layer "F.Cu") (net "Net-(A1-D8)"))
 (segment (start 142.32 136.05) (end 142.32 128.68) (width 0.7) (layer "F.Cu") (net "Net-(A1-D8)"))
 (segment (start 130.75 126.81) (end 130.75 123.185) (width 0.7) (layer "F.Cu") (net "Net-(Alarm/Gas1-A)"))
 (segment (start 130.75 123.185) (end 134.985 118.95) (width 0.7) (layer "F.Cu") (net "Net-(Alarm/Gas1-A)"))
 (segment (start 123.7 135.45) (end 127.26 139.01) (width 0.7) (layer "F.Cu") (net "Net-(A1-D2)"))
 (segment (start 127.26 139.01) (end 127.26 143.435) (width 0.7) (layer "F.Cu") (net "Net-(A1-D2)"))
 (segment (start 142.3 115.22) (end 142.22 115.3) (width 0.7) (layer "F.Cu") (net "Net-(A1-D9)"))
 (segment (start 146.525 120.125) (end 146.525 119.605) (width 0.7) (layer "F.Cu") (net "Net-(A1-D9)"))
 (segment (start 146.56 143.435) (end 146.56 120.16) (width 0.7) (layer "F.Cu") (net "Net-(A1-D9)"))
 (segment (start 146.56 120.16) (end 146.525 120.125) (width 0.7) (layer "F.Cu") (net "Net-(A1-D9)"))
 (segment (start 146.525 119.605) (end 142.22 115.3) (width 0.7) (layer "F.Cu") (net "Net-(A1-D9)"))
 (segment (start 142.3 107.725) (end 142.3 115.22) (width 0.7) (layer "F.Cu") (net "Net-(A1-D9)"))
 (segment (start 131 111.95) (end 134.955 111.95) (width 0.7) (layer "F.Cu") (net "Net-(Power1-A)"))
 (segment (start 134.955 111.95) (end 135.005 112) (width 0.7) (layer "F.Cu") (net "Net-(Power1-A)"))
 (segment (start 130.75 119.19) (end 129.4 120.54) (width 0.7) (layer "F.Cu") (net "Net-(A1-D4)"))
 (segment (start 129.4 120.54) (end 129.4 140.495) (width 0.7) (layer "F.Cu") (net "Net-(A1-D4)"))
 (segment (start 129.4 140.495) (end 132.34 143.435) (width 0.7) (layer "F.Cu") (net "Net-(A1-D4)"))
 (segment (start 128.3 141.935) (end 128.3 107.03) (width 0.7) (layer "F.Cu") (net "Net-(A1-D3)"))
 (segment (start 129.8 143.435) (end 128.3 141.935) (width 0.7) (layer "F.Cu") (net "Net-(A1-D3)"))
 (segment (start 128.3 107.03) (end 131 104.33) (width 0.7) (layer "F.Cu") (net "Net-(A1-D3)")))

